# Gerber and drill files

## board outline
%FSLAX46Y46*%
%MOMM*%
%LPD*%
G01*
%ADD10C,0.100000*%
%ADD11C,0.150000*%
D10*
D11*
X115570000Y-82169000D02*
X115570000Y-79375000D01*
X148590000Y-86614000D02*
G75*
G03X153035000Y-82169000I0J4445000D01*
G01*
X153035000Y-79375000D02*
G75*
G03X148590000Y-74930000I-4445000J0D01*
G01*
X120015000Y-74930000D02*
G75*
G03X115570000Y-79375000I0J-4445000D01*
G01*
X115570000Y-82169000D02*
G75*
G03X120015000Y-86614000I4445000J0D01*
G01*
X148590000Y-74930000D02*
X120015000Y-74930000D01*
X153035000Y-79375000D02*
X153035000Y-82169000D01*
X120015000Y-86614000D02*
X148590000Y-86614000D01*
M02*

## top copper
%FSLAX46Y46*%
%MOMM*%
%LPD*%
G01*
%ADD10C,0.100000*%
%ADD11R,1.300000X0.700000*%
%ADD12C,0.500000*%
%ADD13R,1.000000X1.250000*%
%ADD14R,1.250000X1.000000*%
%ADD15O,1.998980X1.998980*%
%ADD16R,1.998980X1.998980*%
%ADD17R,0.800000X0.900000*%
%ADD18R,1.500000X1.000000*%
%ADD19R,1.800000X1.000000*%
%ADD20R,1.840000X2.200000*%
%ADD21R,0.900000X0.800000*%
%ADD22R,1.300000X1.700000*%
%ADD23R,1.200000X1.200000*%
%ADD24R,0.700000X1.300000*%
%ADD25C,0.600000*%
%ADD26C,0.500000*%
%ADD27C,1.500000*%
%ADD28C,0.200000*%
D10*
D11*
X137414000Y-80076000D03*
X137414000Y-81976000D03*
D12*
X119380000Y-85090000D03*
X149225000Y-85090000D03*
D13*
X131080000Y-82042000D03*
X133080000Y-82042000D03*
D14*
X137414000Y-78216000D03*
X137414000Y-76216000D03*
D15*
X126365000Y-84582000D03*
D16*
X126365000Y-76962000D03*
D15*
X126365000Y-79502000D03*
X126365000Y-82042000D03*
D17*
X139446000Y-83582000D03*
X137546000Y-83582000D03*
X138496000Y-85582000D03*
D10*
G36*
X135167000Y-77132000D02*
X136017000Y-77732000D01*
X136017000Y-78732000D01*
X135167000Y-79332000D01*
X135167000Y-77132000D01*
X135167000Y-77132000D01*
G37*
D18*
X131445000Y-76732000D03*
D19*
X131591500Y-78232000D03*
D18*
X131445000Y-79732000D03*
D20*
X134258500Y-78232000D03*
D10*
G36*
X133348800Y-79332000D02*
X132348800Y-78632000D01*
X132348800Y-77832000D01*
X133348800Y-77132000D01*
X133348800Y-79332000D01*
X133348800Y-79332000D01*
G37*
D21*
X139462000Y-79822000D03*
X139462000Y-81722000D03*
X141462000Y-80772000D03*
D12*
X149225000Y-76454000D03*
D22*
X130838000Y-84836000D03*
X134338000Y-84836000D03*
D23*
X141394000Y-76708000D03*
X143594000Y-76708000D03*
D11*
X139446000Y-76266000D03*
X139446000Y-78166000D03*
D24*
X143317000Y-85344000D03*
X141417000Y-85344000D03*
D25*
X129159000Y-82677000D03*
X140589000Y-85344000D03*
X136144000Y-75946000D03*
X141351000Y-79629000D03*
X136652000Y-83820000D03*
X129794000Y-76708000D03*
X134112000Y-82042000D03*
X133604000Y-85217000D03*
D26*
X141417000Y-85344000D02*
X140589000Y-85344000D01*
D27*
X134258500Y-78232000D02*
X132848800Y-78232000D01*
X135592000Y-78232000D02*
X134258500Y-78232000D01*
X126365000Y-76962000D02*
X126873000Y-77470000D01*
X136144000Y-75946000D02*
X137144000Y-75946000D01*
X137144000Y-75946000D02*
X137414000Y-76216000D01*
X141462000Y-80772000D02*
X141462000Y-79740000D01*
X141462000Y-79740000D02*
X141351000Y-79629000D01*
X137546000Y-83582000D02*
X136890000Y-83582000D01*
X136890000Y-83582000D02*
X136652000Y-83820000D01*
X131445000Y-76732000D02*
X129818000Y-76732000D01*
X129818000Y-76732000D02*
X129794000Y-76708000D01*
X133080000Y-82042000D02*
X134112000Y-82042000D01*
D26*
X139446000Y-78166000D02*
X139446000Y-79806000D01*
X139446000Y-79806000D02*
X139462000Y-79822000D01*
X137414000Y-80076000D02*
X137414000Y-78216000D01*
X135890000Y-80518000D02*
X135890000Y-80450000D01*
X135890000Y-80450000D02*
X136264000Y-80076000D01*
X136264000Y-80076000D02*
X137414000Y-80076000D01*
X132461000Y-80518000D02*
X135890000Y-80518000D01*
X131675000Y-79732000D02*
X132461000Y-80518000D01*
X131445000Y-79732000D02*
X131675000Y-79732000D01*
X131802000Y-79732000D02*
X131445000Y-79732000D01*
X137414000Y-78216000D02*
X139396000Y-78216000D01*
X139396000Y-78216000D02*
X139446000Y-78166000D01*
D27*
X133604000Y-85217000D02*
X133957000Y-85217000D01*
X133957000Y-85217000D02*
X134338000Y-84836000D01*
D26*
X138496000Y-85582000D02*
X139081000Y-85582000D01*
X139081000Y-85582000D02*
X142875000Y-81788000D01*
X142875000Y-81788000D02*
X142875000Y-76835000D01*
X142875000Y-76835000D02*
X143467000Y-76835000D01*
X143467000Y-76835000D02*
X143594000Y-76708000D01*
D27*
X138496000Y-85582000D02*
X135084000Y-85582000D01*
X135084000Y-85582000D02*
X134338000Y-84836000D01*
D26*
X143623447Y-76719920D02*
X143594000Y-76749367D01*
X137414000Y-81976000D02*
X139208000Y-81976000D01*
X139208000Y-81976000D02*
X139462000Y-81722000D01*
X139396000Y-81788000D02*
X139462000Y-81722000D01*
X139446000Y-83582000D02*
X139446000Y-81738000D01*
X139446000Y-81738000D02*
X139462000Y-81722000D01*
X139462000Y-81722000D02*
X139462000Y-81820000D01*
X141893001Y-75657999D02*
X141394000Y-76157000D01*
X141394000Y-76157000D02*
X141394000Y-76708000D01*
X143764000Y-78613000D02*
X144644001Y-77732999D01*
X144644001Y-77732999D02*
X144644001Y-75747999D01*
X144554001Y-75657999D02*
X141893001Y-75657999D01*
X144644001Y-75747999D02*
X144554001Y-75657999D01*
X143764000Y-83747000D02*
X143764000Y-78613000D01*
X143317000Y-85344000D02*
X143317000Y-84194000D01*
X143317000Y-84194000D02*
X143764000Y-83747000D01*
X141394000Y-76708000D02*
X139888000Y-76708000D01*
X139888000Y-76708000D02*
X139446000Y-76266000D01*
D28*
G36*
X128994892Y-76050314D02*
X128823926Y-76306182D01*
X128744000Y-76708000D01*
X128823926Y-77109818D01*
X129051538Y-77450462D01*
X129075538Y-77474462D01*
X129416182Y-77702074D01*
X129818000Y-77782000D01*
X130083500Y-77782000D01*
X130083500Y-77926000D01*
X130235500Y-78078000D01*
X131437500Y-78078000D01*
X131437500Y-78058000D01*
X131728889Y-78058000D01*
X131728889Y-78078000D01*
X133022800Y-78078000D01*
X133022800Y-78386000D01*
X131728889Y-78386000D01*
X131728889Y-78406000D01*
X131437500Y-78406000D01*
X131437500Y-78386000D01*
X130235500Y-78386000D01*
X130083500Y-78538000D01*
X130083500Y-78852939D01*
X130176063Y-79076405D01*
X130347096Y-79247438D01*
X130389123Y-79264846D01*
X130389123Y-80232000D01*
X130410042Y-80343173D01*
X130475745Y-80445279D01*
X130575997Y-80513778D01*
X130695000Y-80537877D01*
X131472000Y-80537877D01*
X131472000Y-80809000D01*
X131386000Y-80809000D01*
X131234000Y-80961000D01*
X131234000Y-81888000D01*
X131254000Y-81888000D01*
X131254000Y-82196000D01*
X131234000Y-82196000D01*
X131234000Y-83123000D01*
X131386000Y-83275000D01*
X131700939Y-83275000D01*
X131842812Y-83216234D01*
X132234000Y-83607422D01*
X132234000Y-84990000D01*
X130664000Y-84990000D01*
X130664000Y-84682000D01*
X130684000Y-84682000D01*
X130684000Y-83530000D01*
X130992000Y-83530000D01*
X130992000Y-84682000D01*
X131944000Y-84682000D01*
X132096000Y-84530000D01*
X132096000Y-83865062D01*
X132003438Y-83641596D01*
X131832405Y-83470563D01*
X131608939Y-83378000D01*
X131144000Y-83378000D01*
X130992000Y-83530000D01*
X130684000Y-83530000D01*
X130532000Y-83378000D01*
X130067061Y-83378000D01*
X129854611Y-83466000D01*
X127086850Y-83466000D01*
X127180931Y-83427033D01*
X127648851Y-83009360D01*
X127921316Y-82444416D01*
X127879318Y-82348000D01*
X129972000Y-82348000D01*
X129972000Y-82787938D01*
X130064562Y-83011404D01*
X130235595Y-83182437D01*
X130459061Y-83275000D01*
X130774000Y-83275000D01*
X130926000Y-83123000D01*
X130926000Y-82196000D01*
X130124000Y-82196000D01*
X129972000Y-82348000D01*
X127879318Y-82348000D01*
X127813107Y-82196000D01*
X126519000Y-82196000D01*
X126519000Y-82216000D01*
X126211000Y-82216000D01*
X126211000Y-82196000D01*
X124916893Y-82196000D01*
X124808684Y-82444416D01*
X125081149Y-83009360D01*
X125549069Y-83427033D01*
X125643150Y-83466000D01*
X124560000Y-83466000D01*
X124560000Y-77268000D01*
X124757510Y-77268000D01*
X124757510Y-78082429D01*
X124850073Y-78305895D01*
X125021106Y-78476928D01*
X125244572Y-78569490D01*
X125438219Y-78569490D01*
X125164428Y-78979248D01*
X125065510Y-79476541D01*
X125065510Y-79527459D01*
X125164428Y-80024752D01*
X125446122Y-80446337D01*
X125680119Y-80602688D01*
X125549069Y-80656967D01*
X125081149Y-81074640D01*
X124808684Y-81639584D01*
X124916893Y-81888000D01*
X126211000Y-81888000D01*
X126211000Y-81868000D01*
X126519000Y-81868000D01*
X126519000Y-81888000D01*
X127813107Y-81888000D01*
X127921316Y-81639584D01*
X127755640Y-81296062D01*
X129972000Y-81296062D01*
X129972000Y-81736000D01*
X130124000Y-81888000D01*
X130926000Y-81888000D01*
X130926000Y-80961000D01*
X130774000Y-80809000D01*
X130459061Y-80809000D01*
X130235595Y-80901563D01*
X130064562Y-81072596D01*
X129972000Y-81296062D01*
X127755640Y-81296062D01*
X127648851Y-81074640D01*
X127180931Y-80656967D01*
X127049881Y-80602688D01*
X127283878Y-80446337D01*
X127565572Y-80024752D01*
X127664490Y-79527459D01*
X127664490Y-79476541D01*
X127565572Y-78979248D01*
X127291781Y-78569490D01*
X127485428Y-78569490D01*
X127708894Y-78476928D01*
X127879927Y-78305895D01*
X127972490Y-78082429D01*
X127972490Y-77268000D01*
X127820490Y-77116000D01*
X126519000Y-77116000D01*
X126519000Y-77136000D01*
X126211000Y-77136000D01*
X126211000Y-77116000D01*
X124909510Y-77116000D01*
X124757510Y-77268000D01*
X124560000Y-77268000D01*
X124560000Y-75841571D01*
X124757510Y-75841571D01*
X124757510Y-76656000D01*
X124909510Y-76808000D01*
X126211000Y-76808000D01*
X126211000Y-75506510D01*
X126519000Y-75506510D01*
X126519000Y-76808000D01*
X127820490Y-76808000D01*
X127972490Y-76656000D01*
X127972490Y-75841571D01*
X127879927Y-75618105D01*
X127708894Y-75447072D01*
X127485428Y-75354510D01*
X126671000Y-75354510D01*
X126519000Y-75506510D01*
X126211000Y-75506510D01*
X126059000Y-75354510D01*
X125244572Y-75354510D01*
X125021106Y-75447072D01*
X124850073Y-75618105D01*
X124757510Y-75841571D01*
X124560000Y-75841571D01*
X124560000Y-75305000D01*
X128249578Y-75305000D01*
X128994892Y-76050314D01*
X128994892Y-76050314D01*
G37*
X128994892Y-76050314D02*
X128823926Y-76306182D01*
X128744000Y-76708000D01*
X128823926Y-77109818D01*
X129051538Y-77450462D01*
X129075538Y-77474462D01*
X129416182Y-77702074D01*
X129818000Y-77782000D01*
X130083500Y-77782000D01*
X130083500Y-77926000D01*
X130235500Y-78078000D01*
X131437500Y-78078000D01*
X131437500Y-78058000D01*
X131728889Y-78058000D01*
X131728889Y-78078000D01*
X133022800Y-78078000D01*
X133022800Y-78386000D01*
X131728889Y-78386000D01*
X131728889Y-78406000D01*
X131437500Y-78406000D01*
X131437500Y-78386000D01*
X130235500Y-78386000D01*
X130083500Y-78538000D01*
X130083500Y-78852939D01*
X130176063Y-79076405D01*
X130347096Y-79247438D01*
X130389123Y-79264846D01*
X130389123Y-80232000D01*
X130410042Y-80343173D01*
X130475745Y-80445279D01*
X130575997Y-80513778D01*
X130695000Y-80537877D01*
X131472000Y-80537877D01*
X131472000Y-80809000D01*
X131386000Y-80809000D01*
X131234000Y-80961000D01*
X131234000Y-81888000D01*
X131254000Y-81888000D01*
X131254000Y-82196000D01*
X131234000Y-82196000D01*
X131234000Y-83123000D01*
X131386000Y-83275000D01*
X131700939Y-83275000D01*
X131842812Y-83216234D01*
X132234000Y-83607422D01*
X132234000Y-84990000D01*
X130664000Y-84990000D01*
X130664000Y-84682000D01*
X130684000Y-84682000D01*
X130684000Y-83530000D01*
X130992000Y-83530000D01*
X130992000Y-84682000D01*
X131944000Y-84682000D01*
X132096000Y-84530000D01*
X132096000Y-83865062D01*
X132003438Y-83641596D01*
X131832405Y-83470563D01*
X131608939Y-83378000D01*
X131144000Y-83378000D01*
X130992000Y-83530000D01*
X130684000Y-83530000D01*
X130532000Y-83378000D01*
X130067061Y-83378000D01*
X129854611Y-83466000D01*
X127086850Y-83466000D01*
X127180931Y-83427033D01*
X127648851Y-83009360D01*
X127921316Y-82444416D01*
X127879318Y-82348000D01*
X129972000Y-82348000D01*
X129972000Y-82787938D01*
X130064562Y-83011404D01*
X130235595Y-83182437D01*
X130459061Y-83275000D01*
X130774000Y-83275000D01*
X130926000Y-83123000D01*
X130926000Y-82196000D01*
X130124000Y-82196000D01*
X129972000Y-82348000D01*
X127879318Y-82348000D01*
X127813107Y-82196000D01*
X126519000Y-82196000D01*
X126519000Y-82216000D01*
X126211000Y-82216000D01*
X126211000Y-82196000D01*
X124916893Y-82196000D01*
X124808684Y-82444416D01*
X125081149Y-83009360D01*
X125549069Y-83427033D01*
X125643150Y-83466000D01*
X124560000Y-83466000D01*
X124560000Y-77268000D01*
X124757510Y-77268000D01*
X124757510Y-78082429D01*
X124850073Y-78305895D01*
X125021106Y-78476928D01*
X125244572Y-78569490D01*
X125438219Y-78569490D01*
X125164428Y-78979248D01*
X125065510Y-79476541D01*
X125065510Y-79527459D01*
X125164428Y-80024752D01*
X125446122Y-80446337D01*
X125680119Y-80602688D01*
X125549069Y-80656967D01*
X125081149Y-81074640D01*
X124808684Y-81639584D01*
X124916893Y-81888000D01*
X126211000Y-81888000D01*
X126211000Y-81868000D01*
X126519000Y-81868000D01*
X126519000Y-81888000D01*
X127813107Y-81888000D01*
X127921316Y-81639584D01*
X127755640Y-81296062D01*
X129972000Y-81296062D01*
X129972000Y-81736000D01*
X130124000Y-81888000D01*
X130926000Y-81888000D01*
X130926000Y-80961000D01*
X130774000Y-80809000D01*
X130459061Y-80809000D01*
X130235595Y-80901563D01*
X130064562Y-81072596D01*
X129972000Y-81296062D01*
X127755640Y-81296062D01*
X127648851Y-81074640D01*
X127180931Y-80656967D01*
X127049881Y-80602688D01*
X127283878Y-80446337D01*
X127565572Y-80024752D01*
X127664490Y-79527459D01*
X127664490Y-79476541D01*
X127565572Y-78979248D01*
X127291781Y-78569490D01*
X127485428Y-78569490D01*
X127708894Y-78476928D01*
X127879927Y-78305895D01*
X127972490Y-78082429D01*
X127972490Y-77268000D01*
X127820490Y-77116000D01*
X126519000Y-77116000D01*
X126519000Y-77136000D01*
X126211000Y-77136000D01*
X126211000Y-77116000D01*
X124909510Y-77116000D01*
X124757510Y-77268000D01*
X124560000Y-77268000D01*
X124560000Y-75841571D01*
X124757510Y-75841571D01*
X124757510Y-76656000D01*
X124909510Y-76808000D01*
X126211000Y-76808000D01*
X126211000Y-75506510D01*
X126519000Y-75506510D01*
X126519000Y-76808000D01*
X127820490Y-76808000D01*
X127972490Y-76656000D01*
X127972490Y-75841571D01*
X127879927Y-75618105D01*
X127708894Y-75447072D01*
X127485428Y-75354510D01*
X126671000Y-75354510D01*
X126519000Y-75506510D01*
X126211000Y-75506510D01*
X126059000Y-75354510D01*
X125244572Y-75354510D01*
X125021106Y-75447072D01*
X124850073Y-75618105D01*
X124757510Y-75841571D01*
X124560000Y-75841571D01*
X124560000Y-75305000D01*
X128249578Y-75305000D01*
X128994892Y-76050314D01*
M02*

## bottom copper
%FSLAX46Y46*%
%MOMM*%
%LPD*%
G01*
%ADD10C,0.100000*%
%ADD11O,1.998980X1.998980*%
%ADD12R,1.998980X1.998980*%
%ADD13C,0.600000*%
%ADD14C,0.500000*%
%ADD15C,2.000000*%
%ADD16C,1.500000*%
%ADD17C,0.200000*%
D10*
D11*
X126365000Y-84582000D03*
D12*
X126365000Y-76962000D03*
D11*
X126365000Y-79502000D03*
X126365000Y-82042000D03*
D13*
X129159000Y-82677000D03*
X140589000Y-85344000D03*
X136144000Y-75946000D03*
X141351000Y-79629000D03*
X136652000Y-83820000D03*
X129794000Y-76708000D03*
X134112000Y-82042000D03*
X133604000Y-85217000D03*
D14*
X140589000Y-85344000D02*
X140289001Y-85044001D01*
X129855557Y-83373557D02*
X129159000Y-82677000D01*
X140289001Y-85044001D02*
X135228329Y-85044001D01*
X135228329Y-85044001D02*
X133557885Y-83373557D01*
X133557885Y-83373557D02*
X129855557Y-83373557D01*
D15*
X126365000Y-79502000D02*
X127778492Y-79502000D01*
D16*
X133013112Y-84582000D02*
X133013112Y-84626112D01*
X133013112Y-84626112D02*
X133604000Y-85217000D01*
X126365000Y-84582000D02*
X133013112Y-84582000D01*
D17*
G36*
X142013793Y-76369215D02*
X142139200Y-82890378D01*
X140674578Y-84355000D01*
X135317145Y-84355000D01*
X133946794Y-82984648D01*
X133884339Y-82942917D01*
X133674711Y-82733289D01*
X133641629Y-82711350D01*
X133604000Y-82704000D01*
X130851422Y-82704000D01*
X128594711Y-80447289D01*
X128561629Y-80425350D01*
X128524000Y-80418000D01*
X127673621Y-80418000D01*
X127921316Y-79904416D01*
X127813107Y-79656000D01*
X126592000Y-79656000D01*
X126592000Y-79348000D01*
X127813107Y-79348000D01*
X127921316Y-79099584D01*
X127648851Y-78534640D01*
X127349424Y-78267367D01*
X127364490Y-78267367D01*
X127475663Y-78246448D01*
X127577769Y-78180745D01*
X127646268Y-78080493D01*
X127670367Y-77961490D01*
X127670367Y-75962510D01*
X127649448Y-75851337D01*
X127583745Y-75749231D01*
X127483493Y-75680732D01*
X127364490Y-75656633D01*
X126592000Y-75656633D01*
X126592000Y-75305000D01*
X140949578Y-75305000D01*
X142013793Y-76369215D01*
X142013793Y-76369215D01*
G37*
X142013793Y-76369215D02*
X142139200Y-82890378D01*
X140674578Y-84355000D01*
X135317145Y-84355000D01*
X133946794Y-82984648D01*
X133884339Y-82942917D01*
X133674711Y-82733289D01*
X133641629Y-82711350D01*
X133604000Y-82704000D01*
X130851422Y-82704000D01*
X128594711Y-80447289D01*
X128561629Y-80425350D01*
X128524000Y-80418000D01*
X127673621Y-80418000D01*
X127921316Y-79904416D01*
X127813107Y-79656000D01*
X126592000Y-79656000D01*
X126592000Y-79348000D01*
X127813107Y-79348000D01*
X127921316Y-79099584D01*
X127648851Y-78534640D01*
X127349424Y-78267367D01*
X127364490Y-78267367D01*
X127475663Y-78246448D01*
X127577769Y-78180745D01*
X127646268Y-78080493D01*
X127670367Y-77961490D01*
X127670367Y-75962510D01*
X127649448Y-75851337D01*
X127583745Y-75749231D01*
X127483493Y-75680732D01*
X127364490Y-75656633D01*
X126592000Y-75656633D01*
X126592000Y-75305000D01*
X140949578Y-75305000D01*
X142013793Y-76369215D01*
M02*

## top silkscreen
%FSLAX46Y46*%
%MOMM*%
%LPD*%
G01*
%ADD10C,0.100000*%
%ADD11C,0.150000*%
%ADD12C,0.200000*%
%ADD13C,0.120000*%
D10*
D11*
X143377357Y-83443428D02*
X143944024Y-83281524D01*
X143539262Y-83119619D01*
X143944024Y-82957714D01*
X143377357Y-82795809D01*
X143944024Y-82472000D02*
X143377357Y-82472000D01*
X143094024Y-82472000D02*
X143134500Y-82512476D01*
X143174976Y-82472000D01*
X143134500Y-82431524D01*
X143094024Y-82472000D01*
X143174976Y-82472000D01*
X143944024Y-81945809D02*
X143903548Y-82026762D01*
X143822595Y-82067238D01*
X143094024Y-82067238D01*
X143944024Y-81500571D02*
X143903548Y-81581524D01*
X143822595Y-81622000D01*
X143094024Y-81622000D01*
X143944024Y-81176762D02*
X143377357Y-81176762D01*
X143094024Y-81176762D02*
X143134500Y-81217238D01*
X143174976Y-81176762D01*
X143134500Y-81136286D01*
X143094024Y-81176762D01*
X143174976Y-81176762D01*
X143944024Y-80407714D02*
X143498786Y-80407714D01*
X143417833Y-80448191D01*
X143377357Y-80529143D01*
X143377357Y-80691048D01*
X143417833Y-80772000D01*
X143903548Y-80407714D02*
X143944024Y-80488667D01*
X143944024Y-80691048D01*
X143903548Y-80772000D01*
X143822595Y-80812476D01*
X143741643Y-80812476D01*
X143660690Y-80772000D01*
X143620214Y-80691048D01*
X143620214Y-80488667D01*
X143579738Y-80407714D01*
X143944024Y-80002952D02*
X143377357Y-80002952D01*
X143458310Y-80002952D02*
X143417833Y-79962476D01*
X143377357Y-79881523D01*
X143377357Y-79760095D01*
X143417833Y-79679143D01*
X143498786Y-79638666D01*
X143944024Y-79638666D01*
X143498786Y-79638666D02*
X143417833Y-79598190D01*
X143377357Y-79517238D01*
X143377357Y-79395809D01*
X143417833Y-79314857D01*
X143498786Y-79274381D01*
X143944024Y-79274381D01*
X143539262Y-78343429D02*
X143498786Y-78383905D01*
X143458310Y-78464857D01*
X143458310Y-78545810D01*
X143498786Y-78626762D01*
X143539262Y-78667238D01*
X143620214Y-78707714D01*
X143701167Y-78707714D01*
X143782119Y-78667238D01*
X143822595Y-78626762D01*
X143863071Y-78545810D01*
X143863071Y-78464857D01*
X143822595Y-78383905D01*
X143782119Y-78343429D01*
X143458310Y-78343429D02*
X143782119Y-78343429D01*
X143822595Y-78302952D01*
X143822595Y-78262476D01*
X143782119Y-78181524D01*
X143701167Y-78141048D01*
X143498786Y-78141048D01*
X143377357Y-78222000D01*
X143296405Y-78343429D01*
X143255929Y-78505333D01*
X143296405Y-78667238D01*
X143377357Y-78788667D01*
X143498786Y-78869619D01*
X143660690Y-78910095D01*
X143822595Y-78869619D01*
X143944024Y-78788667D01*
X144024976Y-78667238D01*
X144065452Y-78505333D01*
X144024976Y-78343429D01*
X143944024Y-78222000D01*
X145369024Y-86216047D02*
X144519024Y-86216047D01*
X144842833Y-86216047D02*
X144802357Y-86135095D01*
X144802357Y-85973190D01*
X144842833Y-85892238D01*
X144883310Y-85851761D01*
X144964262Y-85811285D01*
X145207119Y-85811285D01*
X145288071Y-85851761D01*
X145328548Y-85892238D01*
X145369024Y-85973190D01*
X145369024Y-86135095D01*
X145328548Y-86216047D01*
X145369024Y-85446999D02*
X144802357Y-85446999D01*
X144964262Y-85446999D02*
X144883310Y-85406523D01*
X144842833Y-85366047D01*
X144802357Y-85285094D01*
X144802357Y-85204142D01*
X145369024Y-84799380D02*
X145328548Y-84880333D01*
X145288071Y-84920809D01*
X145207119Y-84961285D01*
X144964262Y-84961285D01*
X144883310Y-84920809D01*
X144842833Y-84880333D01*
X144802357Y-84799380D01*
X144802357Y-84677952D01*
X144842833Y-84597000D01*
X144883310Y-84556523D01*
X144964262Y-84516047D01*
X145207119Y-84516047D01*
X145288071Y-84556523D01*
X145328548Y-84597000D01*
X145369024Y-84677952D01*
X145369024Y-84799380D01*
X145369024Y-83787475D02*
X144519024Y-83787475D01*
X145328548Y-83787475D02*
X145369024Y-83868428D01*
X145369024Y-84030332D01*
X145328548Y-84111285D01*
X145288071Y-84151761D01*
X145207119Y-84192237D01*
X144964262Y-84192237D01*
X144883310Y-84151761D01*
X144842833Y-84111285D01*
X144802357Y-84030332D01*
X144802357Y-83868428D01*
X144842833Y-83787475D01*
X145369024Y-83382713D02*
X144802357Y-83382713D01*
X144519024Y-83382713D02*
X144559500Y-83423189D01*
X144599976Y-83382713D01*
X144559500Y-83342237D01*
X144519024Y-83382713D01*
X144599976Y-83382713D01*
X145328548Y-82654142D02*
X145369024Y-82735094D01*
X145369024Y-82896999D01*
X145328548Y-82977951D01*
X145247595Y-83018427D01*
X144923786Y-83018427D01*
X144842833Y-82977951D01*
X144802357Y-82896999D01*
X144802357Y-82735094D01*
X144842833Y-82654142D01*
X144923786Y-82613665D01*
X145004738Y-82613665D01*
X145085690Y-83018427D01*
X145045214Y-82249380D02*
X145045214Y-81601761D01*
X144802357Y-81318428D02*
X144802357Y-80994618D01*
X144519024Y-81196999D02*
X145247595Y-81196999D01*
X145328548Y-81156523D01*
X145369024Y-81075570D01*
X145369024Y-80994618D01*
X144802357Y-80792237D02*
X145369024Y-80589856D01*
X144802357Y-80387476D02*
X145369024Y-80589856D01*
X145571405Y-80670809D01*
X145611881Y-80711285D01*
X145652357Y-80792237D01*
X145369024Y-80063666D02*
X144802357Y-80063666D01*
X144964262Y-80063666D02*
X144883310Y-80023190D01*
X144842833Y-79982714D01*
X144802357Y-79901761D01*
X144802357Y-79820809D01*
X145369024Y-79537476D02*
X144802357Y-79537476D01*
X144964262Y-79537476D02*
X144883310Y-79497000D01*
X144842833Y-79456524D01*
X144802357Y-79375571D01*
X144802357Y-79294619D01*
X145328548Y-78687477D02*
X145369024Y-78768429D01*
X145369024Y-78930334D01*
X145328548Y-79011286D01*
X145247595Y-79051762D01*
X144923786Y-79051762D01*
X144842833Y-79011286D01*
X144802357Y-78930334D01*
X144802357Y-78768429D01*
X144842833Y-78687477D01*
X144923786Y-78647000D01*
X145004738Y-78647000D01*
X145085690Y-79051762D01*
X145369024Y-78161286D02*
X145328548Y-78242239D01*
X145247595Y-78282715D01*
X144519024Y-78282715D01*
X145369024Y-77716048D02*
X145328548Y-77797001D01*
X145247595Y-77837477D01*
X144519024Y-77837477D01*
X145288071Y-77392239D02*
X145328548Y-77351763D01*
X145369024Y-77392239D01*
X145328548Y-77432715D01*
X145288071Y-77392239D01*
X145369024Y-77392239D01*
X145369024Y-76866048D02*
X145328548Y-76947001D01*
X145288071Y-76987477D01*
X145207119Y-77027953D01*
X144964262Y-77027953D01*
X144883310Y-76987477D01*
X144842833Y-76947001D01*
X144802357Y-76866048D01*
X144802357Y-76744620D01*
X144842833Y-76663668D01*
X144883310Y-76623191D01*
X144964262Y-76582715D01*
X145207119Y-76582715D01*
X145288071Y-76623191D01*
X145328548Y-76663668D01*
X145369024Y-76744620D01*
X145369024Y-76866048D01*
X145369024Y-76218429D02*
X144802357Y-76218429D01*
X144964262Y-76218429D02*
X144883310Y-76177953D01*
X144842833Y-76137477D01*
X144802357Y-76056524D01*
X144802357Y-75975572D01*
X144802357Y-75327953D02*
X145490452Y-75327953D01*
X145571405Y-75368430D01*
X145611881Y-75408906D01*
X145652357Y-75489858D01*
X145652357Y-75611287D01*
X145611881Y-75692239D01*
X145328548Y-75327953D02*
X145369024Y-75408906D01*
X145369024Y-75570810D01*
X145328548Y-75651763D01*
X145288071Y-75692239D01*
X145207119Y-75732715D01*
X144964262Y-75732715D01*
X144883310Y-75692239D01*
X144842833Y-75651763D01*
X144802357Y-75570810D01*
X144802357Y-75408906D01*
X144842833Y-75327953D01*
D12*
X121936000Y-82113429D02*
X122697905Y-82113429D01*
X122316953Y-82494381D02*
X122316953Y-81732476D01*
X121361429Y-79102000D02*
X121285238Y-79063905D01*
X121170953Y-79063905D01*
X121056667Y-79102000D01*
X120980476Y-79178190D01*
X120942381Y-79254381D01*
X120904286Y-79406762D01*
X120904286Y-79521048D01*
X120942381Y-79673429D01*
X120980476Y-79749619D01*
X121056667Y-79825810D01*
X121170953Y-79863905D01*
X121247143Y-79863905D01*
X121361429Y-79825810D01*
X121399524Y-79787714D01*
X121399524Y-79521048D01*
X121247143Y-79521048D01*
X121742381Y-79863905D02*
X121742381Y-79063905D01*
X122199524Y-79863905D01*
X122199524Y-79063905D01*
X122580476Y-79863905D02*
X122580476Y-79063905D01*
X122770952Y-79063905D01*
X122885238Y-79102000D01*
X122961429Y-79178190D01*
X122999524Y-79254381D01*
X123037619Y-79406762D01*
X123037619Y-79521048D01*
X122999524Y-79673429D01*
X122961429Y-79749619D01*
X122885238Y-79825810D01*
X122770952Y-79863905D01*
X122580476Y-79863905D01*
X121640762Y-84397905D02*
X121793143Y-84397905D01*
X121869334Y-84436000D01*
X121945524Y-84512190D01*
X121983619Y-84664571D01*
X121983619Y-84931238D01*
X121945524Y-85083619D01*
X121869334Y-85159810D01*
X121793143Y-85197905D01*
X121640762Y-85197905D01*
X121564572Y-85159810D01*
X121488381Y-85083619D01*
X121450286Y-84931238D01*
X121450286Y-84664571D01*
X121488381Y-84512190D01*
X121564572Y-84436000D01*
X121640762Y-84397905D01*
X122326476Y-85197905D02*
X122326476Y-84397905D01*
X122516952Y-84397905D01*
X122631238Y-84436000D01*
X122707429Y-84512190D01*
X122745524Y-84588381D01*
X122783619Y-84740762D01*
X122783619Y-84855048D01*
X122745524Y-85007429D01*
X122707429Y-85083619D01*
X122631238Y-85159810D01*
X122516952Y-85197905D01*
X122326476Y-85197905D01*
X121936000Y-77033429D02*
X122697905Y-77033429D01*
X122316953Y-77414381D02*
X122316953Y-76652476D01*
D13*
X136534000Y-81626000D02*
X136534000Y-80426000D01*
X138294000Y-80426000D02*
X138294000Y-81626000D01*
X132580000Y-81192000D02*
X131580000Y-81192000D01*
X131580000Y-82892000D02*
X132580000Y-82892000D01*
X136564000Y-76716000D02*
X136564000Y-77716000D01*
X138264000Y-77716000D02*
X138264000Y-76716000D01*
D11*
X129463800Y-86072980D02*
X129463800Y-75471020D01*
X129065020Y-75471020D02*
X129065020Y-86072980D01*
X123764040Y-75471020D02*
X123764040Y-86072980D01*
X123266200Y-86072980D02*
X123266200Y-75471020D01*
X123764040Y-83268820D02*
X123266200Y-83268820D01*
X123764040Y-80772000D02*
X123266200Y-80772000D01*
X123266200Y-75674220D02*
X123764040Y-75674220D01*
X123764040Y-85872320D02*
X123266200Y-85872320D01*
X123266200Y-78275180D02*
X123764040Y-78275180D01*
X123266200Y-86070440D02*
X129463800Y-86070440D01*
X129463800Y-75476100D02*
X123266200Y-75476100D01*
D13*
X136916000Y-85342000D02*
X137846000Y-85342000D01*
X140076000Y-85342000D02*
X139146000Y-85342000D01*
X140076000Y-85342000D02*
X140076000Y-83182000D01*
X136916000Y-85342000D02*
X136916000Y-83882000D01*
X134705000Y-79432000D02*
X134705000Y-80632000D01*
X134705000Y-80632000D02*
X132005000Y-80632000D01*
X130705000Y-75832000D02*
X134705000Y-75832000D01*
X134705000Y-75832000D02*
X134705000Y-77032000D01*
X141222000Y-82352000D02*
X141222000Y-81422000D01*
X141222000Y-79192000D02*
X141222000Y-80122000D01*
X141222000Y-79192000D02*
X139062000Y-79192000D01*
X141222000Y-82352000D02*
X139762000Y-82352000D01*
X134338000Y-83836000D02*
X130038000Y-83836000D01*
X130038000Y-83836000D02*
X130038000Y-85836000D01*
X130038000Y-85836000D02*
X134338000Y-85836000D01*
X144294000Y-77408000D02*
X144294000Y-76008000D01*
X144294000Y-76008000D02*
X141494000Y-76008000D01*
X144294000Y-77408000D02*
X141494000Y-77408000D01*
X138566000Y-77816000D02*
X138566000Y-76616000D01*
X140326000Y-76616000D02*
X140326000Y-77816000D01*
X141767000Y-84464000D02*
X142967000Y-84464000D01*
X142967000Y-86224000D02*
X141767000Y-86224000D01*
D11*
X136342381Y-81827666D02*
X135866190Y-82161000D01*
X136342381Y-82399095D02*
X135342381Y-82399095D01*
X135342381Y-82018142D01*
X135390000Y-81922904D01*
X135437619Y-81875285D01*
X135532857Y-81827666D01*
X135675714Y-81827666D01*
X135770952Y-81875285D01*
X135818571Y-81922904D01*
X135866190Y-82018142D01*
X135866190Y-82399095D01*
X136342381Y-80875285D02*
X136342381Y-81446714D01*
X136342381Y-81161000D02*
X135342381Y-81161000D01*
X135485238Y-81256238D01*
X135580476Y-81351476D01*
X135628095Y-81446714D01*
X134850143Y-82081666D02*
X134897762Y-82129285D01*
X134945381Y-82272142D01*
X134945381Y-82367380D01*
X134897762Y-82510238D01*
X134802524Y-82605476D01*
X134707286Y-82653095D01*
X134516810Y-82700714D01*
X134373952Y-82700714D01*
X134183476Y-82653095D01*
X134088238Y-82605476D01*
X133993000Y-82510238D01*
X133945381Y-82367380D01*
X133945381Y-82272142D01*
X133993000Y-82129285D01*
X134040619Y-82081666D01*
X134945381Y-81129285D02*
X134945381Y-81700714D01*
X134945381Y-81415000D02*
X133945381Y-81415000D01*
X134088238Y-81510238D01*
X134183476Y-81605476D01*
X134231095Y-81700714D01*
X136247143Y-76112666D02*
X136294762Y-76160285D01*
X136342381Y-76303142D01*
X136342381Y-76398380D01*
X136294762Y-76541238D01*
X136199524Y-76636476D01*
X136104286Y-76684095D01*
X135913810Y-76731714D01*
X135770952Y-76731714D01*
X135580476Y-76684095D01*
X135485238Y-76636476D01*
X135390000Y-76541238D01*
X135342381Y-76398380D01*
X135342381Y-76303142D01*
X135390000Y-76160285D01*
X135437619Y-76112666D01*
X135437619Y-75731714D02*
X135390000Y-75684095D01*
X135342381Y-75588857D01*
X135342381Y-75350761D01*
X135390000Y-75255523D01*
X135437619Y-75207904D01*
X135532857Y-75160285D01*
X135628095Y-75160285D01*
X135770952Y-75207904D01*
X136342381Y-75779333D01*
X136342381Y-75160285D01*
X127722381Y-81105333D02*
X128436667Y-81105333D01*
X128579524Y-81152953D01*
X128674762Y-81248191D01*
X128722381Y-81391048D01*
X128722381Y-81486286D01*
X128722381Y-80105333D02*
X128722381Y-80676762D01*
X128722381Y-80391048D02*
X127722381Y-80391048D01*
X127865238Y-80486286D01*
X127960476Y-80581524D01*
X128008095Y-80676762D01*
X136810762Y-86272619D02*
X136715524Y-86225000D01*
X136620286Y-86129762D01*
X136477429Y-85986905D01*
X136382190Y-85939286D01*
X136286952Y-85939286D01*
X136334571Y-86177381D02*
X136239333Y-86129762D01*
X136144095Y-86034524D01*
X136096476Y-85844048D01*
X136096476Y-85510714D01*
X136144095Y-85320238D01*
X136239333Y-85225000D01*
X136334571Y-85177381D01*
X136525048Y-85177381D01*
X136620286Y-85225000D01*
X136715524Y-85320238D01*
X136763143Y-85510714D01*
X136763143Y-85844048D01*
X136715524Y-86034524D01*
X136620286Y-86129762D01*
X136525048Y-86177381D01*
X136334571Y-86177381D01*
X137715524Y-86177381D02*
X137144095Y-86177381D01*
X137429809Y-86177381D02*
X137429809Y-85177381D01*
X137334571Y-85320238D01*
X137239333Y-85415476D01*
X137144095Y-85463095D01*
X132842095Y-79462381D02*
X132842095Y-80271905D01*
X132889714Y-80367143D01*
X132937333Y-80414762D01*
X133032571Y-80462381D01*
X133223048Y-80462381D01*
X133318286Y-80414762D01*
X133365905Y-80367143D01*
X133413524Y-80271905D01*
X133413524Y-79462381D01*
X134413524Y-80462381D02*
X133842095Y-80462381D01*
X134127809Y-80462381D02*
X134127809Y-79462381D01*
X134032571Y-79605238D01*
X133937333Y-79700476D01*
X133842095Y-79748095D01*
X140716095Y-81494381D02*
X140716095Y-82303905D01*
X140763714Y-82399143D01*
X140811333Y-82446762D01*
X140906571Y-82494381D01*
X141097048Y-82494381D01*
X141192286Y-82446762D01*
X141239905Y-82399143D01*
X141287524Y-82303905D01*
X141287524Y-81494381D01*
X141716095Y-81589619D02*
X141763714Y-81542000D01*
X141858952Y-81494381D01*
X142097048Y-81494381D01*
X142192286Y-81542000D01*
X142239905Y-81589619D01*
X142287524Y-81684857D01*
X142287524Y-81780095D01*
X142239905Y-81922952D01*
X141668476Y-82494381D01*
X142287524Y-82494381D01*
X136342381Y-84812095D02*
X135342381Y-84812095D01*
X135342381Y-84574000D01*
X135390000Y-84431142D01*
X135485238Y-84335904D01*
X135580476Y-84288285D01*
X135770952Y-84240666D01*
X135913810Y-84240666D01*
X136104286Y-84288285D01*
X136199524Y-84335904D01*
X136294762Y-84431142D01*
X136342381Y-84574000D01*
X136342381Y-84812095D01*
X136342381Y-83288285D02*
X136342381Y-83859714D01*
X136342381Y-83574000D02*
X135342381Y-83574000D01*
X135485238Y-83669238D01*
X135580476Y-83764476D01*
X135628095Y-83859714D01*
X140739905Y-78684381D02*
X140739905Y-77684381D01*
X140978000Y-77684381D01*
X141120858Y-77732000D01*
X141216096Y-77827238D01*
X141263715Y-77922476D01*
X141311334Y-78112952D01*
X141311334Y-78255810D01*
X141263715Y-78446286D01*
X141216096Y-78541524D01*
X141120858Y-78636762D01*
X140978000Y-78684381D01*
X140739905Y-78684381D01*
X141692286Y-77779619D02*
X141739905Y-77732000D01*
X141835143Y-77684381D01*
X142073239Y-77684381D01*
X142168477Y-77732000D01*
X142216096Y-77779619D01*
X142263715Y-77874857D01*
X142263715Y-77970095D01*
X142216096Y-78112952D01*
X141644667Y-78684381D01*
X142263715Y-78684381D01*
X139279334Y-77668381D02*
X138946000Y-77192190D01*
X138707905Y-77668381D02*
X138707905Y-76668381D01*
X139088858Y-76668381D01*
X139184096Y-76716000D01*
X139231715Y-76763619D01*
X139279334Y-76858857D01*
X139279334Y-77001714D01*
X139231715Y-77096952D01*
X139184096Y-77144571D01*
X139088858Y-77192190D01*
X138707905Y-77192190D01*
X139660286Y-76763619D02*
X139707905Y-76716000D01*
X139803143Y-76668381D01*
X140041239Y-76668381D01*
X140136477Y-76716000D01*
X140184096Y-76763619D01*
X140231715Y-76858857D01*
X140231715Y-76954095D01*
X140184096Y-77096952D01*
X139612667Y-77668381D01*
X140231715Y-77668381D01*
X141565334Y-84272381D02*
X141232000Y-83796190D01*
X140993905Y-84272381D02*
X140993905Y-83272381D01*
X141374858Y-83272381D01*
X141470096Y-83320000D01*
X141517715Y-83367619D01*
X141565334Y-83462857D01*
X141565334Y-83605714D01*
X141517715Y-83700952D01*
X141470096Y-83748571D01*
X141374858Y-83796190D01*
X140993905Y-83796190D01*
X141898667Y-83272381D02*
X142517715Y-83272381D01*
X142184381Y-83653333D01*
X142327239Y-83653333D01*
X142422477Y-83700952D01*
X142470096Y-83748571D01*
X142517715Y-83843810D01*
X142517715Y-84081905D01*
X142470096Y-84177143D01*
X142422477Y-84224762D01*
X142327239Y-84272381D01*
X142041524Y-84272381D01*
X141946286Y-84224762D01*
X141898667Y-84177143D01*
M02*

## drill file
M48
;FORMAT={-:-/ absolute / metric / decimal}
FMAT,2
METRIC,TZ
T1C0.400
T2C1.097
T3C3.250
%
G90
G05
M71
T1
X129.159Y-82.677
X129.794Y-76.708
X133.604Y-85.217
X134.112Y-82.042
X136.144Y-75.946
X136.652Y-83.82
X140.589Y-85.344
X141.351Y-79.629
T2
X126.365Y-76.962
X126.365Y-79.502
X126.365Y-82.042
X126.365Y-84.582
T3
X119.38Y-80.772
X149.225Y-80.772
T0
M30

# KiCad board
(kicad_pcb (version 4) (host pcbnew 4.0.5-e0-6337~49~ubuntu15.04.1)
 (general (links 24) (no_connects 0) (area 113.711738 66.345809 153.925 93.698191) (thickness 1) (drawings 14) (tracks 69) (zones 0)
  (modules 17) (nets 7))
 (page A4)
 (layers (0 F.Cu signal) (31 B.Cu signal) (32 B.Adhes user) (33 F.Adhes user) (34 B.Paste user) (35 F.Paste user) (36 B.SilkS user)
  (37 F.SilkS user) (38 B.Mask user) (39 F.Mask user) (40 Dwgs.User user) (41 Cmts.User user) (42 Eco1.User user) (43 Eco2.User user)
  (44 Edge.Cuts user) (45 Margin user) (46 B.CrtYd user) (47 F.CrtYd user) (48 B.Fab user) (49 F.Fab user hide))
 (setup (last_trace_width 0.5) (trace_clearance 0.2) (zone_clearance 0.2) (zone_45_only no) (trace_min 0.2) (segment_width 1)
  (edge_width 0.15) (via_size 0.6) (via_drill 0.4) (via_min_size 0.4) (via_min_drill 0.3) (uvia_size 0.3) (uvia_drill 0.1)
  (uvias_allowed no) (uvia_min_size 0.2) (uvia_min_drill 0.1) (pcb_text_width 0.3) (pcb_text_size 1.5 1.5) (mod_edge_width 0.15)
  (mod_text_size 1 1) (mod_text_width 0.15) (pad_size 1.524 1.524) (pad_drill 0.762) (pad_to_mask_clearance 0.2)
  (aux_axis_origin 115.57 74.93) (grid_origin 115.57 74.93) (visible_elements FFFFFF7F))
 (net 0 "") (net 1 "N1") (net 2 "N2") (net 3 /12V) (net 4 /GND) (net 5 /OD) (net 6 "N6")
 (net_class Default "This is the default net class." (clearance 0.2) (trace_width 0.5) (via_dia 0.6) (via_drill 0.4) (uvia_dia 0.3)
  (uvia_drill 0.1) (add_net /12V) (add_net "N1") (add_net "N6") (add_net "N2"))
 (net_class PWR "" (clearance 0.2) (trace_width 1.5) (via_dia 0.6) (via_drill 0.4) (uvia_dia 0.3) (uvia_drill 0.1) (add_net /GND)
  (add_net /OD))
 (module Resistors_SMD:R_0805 (layer F.Cu) (at 137.414 81.026 270)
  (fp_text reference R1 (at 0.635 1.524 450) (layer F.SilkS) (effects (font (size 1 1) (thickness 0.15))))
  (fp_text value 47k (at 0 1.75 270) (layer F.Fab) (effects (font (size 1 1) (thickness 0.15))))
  (fp_line (start 0.6 0.88) (end -0.6 0.88) (layer F.SilkS) (width 0.12))
  (fp_line (start -0.6 -0.88) (end 0.6 -0.88) (layer F.SilkS) (width 0.12))
  (pad 1 smd rect (at -0.95 0 270) (size 0.7 1.3) (layers F.Cu F.Paste F.Mask) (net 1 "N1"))
  (pad 2 smd rect (at 0.95 0 270) (size 0.7 1.3) (layers F.Cu F.Paste F.Mask) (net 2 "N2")))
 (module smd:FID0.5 (layer F.Cu) (at 119.38 85.09)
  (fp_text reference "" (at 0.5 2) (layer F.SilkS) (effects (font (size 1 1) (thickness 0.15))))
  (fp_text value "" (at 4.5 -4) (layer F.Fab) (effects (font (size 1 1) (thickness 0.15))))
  (pad F smd circle (at 0 0) (size 0.5 0.5) (layers F.Cu F.Mask) (solder_mask_margin 1) (clearance 1)))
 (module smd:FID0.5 (layer F.Cu) (at 149.225 85.09)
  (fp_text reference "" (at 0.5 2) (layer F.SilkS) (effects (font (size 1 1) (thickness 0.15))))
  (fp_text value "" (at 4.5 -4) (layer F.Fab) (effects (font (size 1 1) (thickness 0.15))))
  (pad F smd circle (at 0 0) (size 0.5 0.5) (layers F.Cu F.Mask) (solder_mask_margin 1) (clearance 1)))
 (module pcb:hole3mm (layer F.Cu) (at 149.225 80.772)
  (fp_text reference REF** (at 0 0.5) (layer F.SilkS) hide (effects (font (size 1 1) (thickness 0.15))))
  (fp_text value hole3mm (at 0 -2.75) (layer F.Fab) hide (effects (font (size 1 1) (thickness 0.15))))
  (pad "" np_thru_hole circle (at 0 0) (size 3.25 3.25) (drill 3.25) (layers *.Cu *.Mask) (solder_mask_margin 1.9) (solder_paste_margin 1.9)
   (clearance 1.9)))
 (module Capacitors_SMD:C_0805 (layer F.Cu) (at 132.08 82.042)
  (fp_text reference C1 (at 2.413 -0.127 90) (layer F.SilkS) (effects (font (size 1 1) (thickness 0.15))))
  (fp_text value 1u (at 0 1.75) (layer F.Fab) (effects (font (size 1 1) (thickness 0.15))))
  (fp_line (start 0.5 -0.85) (end -0.5 -0.85) (layer F.SilkS) (width 0.12))
  (fp_line (start -0.5 0.85) (end 0.5 0.85) (layer F.SilkS) (width 0.12))
  (pad 1 smd rect (at -1 0) (size 1 1.25) (layers F.Cu F.Paste F.Mask) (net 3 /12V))
  (pad 2 smd rect (at 1 0) (size 1 1.25) (layers F.Cu F.Paste F.Mask) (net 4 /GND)))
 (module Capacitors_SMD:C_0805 (layer F.Cu) (at 137.414 77.216 90)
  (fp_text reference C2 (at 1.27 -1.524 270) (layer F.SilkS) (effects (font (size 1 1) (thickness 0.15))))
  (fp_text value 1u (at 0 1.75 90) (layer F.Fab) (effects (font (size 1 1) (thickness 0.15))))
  (fp_line (start 0.5 -0.85) (end -0.5 -0.85) (layer F.SilkS) (width 0.12))
  (fp_line (start -0.5 0.85) (end 0.5 0.85) (layer F.SilkS) (width 0.12))
  (pad 1 smd rect (at -1 0 90) (size 1 1.25) (layers F.Cu F.Paste F.Mask) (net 1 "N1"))
  (pad 2 smd rect (at 1 0 90) (size 1 1.25) (layers F.Cu F.Paste F.Mask) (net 4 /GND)))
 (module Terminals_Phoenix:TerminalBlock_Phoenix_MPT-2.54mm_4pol (layer F.Cu) (at 126.365 76.962 270)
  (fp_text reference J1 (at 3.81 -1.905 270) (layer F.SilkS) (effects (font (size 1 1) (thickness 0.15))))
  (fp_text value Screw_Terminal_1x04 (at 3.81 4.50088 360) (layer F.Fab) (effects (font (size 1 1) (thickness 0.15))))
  (fp_line (start 9.11098 -3.0988) (end -1.49098 -3.0988) (layer F.SilkS) (width 0.15))
  (fp_line (start -1.49098 -2.70002) (end 9.11098 -2.70002) (layer F.SilkS) (width 0.15))
  (fp_line (start -1.49098 2.60096) (end 9.11098 2.60096) (layer F.SilkS) (width 0.15))
  (fp_line (start 9.11098 3.0988) (end -1.49098 3.0988) (layer F.SilkS) (width 0.15))
  (fp_line (start 6.30682 2.60096) (end 6.30682 3.0988) (layer F.SilkS) (width 0.15))
  (fp_line (start 3.81 2.60096) (end 3.81 3.0988) (layer F.SilkS) (width 0.15))
  (fp_line (start -1.28778 3.0988) (end -1.28778 2.60096) (layer F.SilkS) (width 0.15))
  (fp_line (start 8.91032 2.60096) (end 8.91032 3.0988) (layer F.SilkS) (width 0.15))
  (fp_line (start 1.31318 3.0988) (end 1.31318 2.60096) (layer F.SilkS) (width 0.15))
  (fp_line (start 9.10844 3.0988) (end 9.10844 -3.0988) (layer F.SilkS) (width 0.15))
  (fp_line (start -1.4859 -3.0988) (end -1.4859 3.0988) (layer F.SilkS) (width 0.15))
  (pad 4 thru_hole oval (at 7.62 0 90) (size 1.99898 1.99898) (drill 1.09728) (layers *.Cu *.Mask) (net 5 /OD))
  (pad 1 thru_hole rect (at 0 0 90) (size 1.99898 1.99898) (drill 1.09728) (layers *.Cu *.Mask) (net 3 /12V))
  (pad 2 thru_hole oval (at 2.54 0 90) (size 1.99898 1.99898) (drill 1.09728) (layers *.Cu *.Mask) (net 4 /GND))
  (pad 3 thru_hole oval (at 5.08 0 90) (size 1.99898 1.99898) (drill 1.09728) (layers *.Cu *.Mask) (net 3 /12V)))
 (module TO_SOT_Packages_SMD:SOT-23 (layer F.Cu) (at 138.496 84.582 270)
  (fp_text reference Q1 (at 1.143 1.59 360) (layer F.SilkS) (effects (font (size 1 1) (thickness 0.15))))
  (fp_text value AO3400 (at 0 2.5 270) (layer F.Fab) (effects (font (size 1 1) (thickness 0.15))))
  (fp_line (start 0.76 1.58) (end 0.76 0.65) (layer F.SilkS) (width 0.12))
  (fp_line (start 0.76 -1.58) (end 0.76 -0.65) (layer F.SilkS) (width 0.12))
  (fp_line (start 0.76 -1.58) (end -1.4 -1.58) (layer F.SilkS) (width 0.12))
  (fp_line (start 0.76 1.58) (end -0.7 1.58) (layer F.SilkS) (width 0.12))
  (pad 1 smd rect (at -1 -0.95 270) (size 0.9 0.8) (layers F.Cu F.Paste F.Mask) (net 2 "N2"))
  (pad 2 smd rect (at -1 0.95 270) (size 0.9 0.8) (layers F.Cu F.Paste F.Mask) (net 4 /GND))
  (pad 3 smd rect (at 1 0 270) (size 0.9 0.8) (layers F.Cu F.Paste F.Mask) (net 5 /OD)))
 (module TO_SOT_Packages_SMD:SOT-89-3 (layer F.Cu) (at 132.925 78.232)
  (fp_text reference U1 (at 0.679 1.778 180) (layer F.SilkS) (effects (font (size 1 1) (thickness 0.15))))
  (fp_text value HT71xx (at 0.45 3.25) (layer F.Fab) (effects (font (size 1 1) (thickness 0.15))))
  (fp_line (start 1.78 1.2) (end 1.78 2.4) (layer F.SilkS) (width 0.12))
  (fp_line (start 1.78 2.4) (end -0.92 2.4) (layer F.SilkS) (width 0.12))
  (fp_line (start -2.22 -2.4) (end 1.78 -2.4) (layer F.SilkS) (width 0.12))
  (fp_line (start 1.78 -2.4) (end 1.78 -1.2) (layer F.SilkS) (width 0.12))
  (pad 2 smd trapezoid (at 2.667 0 270) (size 1.6 0.85) (rect_delta 0 0.6) (layers F.Cu F.Paste F.Mask) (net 3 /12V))
  (pad 1 smd rect (at -1.48 -1.5 270) (size 1 1.5) (layers F.Cu F.Paste F.Mask) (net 4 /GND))
  (pad 2 smd rect (at -1.3335 0 270) (size 1 1.8) (layers F.Cu F.Paste F.Mask) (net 3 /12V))
  (pad 3 smd rect (at -1.48 1.5 270) (size 1 1.5) (layers F.Cu F.Paste F.Mask) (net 1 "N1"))
  (pad 2 smd rect (at 1.3335 0 270) (size 2.2 1.84) (layers F.Cu F.Paste F.Mask) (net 3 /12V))
  (pad 2 smd trapezoid (at -0.0762 0 90) (size 1.5 1) (rect_delta 0 0.7) (layers F.Cu F.Paste F.Mask) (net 3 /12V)))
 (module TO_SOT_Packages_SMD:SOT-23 (layer F.Cu) (at 140.462 80.772)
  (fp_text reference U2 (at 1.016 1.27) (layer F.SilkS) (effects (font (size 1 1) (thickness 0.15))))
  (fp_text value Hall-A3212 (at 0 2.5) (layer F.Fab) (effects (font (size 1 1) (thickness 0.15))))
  (fp_line (start 0.76 1.58) (end 0.76 0.65) (layer F.SilkS) (width 0.12))
  (fp_line (start 0.76 -1.58) (end 0.76 -0.65) (layer F.SilkS) (width 0.12))
  (fp_line (start 0.76 -1.58) (end -1.4 -1.58) (layer F.SilkS) (width 0.12))
  (fp_line (start 0.76 1.58) (end -0.7 1.58) (layer F.SilkS) (width 0.12))
  (pad 1 smd rect (at -1 -0.95) (size 0.9 0.8) (layers F.Cu F.Paste F.Mask) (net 1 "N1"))
  (pad 2 smd rect (at -1 0.95) (size 0.9 0.8) (layers F.Cu F.Paste F.Mask) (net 2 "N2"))
  (pad 3 smd rect (at 1 0) (size 0.9 0.8) (layers F.Cu F.Paste F.Mask) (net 4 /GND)))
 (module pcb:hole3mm (layer F.Cu) (at 119.38 80.772)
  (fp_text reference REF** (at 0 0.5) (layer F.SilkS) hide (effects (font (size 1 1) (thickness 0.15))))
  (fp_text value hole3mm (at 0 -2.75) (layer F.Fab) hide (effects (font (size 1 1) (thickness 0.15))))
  (pad "" np_thru_hole circle (at 0 0) (size 3.25 3.25) (drill 3.25) (layers *.Cu *.Mask) (solder_mask_margin 1.9) (solder_paste_margin 1.9)
   (clearance 1.9)))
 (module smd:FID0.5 (layer F.Cu) (at 149.225 76.454)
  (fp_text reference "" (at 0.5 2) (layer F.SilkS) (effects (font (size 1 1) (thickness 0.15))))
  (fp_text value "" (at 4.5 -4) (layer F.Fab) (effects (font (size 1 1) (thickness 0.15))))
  (pad F smd circle (at 0 0) (size 0.5 0.5) (layers F.Cu F.Mask) (solder_mask_margin 1) (clearance 1)))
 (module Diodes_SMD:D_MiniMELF (layer F.Cu) (at 132.588 84.836)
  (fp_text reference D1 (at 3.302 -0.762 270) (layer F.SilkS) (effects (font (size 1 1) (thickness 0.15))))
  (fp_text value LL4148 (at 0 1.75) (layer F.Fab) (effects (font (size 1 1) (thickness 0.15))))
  (fp_line (start 1.75 -1) (end -2.55 -1) (layer F.SilkS) (width 0.12))
  (fp_line (start -2.55 -1) (end -2.55 1) (layer F.SilkS) (width 0.12))
  (fp_line (start -2.55 1) (end 1.75 1) (layer F.SilkS) (width 0.12))
  (pad 1 smd rect (at -1.75 0) (size 1.3 1.7) (layers F.Cu F.Paste F.Mask) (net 3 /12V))
  (pad 2 smd rect (at 1.75 0) (size 1.3 1.7) (layers F.Cu F.Paste F.Mask) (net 5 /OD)))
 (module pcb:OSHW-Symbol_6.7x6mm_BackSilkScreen (layer F.Cu) (at 140.081 80.772 90)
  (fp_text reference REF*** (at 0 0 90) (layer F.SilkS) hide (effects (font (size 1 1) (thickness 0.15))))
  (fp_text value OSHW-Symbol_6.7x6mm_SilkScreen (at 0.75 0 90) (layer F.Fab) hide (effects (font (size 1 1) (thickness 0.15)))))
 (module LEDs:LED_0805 (layer F.Cu) (at 142.494 76.708 180)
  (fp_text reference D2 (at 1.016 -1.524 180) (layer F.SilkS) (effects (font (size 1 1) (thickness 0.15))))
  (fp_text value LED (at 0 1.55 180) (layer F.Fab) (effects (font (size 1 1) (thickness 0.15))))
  (fp_line (start -1.8 -0.7) (end -1.8 0.7) (layer F.SilkS) (width 0.12))
  (fp_line (start -1.8 0.7) (end 1 0.7) (layer F.SilkS) (width 0.12))
  (fp_line (start -1.8 -0.7) (end 1 -0.7) (layer F.SilkS) (width 0.12))
  (pad 2 smd rect (at 1.1 0) (size 1.2 1.2) (layers F.Cu F.Paste F.Mask) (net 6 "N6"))
  (pad 1 smd rect (at -1.1 0) (size 1.2 1.2) (layers F.Cu F.Paste F.Mask) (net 5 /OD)))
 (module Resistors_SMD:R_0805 (layer F.Cu) (at 139.446 77.216 270)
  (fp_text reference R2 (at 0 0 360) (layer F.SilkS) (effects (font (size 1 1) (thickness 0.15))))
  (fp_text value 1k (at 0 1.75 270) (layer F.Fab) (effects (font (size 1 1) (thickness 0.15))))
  (fp_line (start 0.6 0.88) (end -0.6 0.88) (layer F.SilkS) (width 0.12))
  (fp_line (start -0.6 -0.88) (end 0.6 -0.88) (layer F.SilkS) (width 0.12))
  (pad 1 smd rect (at -0.95 0 270) (size 0.7 1.3) (layers F.Cu F.Paste F.Mask) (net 6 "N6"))
  (pad 2 smd rect (at 0.95 0 270) (size 0.7 1.3) (layers F.Cu F.Paste F.Mask) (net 1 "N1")))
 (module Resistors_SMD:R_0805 (layer F.Cu) (at 142.367 85.344 180)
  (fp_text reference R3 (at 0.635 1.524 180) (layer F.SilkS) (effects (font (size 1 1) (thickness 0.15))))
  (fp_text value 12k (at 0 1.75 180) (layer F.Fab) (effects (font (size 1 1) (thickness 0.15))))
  (fp_line (start 0.6 0.88) (end -0.6 0.88) (layer F.SilkS) (width 0.12))
  (fp_line (start -0.6 -0.88) (end 0.6 -0.88) (layer F.SilkS) (width 0.12))
  (pad 1 smd rect (at -0.95 0 180) (size 0.7 1.3) (layers F.Cu F.Paste F.Mask) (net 6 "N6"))
  (pad 2 smd rect (at 0.95 0 180) (size 0.7 1.3) (layers F.Cu F.Paste F.Mask) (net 3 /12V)))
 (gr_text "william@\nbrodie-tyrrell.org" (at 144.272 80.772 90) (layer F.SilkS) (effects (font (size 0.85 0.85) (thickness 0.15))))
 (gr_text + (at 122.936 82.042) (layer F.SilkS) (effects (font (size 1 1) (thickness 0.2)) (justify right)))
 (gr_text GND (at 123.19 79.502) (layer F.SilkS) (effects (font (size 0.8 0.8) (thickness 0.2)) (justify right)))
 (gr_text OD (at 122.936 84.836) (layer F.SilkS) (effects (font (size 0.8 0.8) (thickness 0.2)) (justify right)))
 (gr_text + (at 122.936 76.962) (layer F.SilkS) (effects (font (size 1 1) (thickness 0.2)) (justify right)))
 (gr_line (start 115.57 82.169) (end 115.57 79.375) (layer Edge.Cuts) (width 0.15))
 (gr_arc (start 148.59 82.169) (end 153.035 82.169) (angle 90) (layer Edge.Cuts) (width 0.15))
 (gr_arc (start 148.59 79.375) (end 148.59 74.93) (angle 90) (layer Edge.Cuts) (width 0.15))
 (gr_arc (start 120.015 79.375) (end 115.57 79.375) (angle 90) (layer Edge.Cuts) (width 0.15))
 (gr_arc (start 120.015 82.169) (end 120.015 86.614) (angle 90) (layer Edge.Cuts) (width 0.15))
 (gr_line (start 148.59 74.93) (end 120.015 74.93) (layer Edge.Cuts) (width 0.15))
 (gr_line (start 153.035 79.375) (end 153.035 82.169) (layer Edge.Cuts) (width 0.15))
 (gr_line (start 120.015 86.614) (end 148.59 86.614) (layer Edge.Cuts) (width 0.15))
 (segment (start 140.589 85.344) (end 140.289001 85.044001) (width 0.5) (layer B.Cu) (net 3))
 (segment (start 129.855557 83.373557) (end 129.159 82.677) (width 0.5) (layer B.Cu) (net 3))
 (segment (start 140.289001 85.044001) (end 135.228329 85.044001) (width 0.5) (layer B.Cu) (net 3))
 (segment (start 135.228329 85.044001) (end 133.557885 83.373557) (width 0.5) (layer B.Cu) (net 3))
 (segment (start 133.557885 83.373557) (end 129.855557 83.373557) (width 0.5) (layer B.Cu) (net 3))
 (via (at 129.159 82.677) (size 0.6) (drill 0.4) (layers F.Cu B.Cu) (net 3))
 (segment (start 141.417 85.344) (end 140.589 85.344) (width 0.5) (layer F.Cu) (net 3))
 (via (at 140.589 85.344) (size 0.6) (drill 0.4) (layers F.Cu B.Cu) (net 3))
 (segment (start 134.2585 78.232) (end 132.8488 78.232) (width 1.5) (layer F.Cu) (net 3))
 (segment (start 135.592 78.232) (end 134.2585 78.232) (width 1.5) (layer F.Cu) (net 3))
 (segment (start 126.365 76.962) (end 126.873 77.47) (width 1.5) (layer F.Cu) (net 3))
 (segment (start 136.144 75.946) (end 137.144 75.946) (width 1.5) (layer F.Cu) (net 4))
 (segment (start 137.144 75.946) (end 137.414 76.216) (width 1.5) (layer F.Cu) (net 4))
 (via (at 136.144 75.946) (size 0.6) (drill 0.4) (layers F.Cu B.Cu) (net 4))
 (segment (start 141.462 80.772) (end 141.462 79.74) (width 1.5) (layer F.Cu) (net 4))
 (segment (start 141.462 79.74) (end 141.351 79.629) (width 1.5) (layer F.Cu) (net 4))
 (via (at 141.351 79.629) (size 0.6) (drill 0.4) (layers F.Cu B.Cu) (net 4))
 (segment (start 137.546 83.582) (end 136.89 83.582) (width 1.5) (layer F.Cu) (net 4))
 (segment (start 136.89 83.582) (end 136.652 83.82) (width 1.5) (layer F.Cu) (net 4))
 (via (at 136.652 83.82) (size 0.6) (drill 0.4) (layers F.Cu B.Cu) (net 4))
 (segment (start 131.445 76.732) (end 129.818 76.732) (width 1.5) (layer F.Cu) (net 4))
 (segment (start 129.818 76.732) (end 129.794 76.708) (width 1.5) (layer F.Cu) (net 4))
 (via (at 129.794 76.708) (size 0.6) (drill 0.4) (layers F.Cu B.Cu) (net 4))
 (segment (start 133.08 82.042) (end 134.112 82.042) (width 1.5) (layer F.Cu) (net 4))
 (via (at 134.112 82.042) (size 0.6) (drill 0.4) (layers F.Cu B.Cu) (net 4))
 (segment (start 126.365 79.502) (end 127.778492 79.502) (width 2) (layer B.Cu) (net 4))
 (segment (start 139.446 78.166) (end 139.446 79.806) (width 0.5) (layer F.Cu) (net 1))
 (segment (start 139.446 79.806) (end 139.462 79.822) (width 0.5) (layer F.Cu) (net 1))
 (segment (start 137.414 80.076) (end 137.414 78.216) (width 0.5) (layer F.Cu) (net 1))
 (segment (start 135.89 80.518) (end 135.89 80.45) (width 0.5) (layer F.Cu) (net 1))
 (segment (start 135.89 80.45) (end 136.264 80.076) (width 0.5) (layer F.Cu) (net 1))
 (segment (start 136.264 80.076) (end 137.414 80.076) (width 0.5) (layer F.Cu) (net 1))
 (segment (start 132.461 80.518) (end 135.89 80.518) (width 0.5) (layer F.Cu) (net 1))
 (segment (start 131.675 79.732) (end 132.461 80.518) (width 0.5) (layer F.Cu) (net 1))
 (segment (start 131.445 79.732) (end 131.675 79.732) (width 0.5) (layer F.Cu) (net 1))
 (segment (start 131.802 79.732) (end 131.445 79.732) (width 0.5) (layer F.Cu) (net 1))
 (segment (start 137.414 78.216) (end 139.396 78.216) (width 0.5) (layer F.Cu) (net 1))
 (segment (start 139.396 78.216) (end 139.446 78.166) (width 0.5) (layer F.Cu) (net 1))
 (segment (start 133.604 85.217) (end 133.957 85.217) (width 1.5) (layer F.Cu) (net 5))
 (segment (start 133.957 85.217) (end 134.338 84.836) (width 1.5) (layer F.Cu) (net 5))
 (segment (start 133.013112 84.582) (end 133.013112 84.626112) (width 1.5) (layer B.Cu) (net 5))
 (segment (start 133.013112 84.626112) (end 133.604 85.217) (width 1.5) (layer B.Cu) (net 5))
 (via (at 133.604 85.217) (size 0.6) (drill 0.4) (layers F.Cu B.Cu) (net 5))
 (segment (start 138.496 85.582) (end 139.081 85.582) (width 0.5) (layer F.Cu) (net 5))
 (segment (start 139.081 85.582) (end 142.875 81.788) (width 0.5) (layer F.Cu) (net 5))
 (segment (start 142.875 81.788) (end 142.875 76.835) (width 0.5) (layer F.Cu) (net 5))
 (segment (start 142.875 76.835) (end 143.467 76.835) (width 0.5) (layer F.Cu) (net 5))
 (segment (start 143.467 76.835) (end 143.594 76.708) (width 0.5) (layer F.Cu) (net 5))
 (segment (start 138.496 85.582) (end 135.084 85.582) (width 1.5) (layer F.Cu) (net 5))
 (segment (start 135.084 85.582) (end 134.338 84.836) (width 1.5) (layer F.Cu) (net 5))
 (segment (start 126.365 84.582) (end 133.013112 84.582) (width 1.5) (layer B.Cu) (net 5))
 (segment (start 143.623447 76.71992) (end 143.594 76.749367) (width 0.5) (layer F.Cu) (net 5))
 (segment (start 137.414 81.976) (end 139.208 81.976) (width 0.5) (layer F.Cu) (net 2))
 (segment (start 139.208 81.976) (end 139.462 81.722) (width 0.5) (layer F.Cu) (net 2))
 (segment (start 139.396 81.788) (end 139.462 81.722) (width 0.5) (layer F.Cu) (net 2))
 (segment (start 139.446 83.582) (end 139.446 81.738) (width 0.5) (layer F.Cu) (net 2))
 (segment (start 139.446 81.738) (end 139.462 81.722) (width 0.5) (layer F.Cu) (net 2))
 (segment (start 139.462 81.722) (end 139.462 81.82) (width 0.5) (layer F.Cu) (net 2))
 (segment (start 141.893001 75.657999) (end 141.394 76.157) (width 0.5) (layer F.Cu) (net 6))
 (segment (start 141.394 76.157) (end 141.394 76.708) (width 0.5) (layer F.Cu) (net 6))
 (segment (start 143.764 78.613) (end 144.644001 77.732999) (width 0.5) (layer F.Cu) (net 6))
 (segment (start 144.644001 77.732999) (end 144.644001 75.747999) (width 0.5) (layer F.Cu) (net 6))
 (segment (start 144.554001 75.657999) (end 141.893001 75.657999) (width 0.5) (layer F.Cu) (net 6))
 (segment (start 144.644001 75.747999) (end 144.554001 75.657999) (width 0.5) (layer F.Cu) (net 6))
 (segment (start 143.764 83.747) (end 143.764 78.613) (width 0.5) (layer F.Cu) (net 6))
 (segment (start 143.317 85.344) (end 143.317 84.194) (width 0.5) (layer F.Cu) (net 6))
 (segment (start 143.317 84.194) (end 143.764 83.747) (width 0.5) (layer F.Cu) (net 6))
 (segment (start 141.394 76.708) (end 139.888 76.708) (width 0.5) (layer F.Cu) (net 6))
 (segment (start 139.888 76.708) (end 139.446 76.266) (width 0.5) (layer F.Cu) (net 6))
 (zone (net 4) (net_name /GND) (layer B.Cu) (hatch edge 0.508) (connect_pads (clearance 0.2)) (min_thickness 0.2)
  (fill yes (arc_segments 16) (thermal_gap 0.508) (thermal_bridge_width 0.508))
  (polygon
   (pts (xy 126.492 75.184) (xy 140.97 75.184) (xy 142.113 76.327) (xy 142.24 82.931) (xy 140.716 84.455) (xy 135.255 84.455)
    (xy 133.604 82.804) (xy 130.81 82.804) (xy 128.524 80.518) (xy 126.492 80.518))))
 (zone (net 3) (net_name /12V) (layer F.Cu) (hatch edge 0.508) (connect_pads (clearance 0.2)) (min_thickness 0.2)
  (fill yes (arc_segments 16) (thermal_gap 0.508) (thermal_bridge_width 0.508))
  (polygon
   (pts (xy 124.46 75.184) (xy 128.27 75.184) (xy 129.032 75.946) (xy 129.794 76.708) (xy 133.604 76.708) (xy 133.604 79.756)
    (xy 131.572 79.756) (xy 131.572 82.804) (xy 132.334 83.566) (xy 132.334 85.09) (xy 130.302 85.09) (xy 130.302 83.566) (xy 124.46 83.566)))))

